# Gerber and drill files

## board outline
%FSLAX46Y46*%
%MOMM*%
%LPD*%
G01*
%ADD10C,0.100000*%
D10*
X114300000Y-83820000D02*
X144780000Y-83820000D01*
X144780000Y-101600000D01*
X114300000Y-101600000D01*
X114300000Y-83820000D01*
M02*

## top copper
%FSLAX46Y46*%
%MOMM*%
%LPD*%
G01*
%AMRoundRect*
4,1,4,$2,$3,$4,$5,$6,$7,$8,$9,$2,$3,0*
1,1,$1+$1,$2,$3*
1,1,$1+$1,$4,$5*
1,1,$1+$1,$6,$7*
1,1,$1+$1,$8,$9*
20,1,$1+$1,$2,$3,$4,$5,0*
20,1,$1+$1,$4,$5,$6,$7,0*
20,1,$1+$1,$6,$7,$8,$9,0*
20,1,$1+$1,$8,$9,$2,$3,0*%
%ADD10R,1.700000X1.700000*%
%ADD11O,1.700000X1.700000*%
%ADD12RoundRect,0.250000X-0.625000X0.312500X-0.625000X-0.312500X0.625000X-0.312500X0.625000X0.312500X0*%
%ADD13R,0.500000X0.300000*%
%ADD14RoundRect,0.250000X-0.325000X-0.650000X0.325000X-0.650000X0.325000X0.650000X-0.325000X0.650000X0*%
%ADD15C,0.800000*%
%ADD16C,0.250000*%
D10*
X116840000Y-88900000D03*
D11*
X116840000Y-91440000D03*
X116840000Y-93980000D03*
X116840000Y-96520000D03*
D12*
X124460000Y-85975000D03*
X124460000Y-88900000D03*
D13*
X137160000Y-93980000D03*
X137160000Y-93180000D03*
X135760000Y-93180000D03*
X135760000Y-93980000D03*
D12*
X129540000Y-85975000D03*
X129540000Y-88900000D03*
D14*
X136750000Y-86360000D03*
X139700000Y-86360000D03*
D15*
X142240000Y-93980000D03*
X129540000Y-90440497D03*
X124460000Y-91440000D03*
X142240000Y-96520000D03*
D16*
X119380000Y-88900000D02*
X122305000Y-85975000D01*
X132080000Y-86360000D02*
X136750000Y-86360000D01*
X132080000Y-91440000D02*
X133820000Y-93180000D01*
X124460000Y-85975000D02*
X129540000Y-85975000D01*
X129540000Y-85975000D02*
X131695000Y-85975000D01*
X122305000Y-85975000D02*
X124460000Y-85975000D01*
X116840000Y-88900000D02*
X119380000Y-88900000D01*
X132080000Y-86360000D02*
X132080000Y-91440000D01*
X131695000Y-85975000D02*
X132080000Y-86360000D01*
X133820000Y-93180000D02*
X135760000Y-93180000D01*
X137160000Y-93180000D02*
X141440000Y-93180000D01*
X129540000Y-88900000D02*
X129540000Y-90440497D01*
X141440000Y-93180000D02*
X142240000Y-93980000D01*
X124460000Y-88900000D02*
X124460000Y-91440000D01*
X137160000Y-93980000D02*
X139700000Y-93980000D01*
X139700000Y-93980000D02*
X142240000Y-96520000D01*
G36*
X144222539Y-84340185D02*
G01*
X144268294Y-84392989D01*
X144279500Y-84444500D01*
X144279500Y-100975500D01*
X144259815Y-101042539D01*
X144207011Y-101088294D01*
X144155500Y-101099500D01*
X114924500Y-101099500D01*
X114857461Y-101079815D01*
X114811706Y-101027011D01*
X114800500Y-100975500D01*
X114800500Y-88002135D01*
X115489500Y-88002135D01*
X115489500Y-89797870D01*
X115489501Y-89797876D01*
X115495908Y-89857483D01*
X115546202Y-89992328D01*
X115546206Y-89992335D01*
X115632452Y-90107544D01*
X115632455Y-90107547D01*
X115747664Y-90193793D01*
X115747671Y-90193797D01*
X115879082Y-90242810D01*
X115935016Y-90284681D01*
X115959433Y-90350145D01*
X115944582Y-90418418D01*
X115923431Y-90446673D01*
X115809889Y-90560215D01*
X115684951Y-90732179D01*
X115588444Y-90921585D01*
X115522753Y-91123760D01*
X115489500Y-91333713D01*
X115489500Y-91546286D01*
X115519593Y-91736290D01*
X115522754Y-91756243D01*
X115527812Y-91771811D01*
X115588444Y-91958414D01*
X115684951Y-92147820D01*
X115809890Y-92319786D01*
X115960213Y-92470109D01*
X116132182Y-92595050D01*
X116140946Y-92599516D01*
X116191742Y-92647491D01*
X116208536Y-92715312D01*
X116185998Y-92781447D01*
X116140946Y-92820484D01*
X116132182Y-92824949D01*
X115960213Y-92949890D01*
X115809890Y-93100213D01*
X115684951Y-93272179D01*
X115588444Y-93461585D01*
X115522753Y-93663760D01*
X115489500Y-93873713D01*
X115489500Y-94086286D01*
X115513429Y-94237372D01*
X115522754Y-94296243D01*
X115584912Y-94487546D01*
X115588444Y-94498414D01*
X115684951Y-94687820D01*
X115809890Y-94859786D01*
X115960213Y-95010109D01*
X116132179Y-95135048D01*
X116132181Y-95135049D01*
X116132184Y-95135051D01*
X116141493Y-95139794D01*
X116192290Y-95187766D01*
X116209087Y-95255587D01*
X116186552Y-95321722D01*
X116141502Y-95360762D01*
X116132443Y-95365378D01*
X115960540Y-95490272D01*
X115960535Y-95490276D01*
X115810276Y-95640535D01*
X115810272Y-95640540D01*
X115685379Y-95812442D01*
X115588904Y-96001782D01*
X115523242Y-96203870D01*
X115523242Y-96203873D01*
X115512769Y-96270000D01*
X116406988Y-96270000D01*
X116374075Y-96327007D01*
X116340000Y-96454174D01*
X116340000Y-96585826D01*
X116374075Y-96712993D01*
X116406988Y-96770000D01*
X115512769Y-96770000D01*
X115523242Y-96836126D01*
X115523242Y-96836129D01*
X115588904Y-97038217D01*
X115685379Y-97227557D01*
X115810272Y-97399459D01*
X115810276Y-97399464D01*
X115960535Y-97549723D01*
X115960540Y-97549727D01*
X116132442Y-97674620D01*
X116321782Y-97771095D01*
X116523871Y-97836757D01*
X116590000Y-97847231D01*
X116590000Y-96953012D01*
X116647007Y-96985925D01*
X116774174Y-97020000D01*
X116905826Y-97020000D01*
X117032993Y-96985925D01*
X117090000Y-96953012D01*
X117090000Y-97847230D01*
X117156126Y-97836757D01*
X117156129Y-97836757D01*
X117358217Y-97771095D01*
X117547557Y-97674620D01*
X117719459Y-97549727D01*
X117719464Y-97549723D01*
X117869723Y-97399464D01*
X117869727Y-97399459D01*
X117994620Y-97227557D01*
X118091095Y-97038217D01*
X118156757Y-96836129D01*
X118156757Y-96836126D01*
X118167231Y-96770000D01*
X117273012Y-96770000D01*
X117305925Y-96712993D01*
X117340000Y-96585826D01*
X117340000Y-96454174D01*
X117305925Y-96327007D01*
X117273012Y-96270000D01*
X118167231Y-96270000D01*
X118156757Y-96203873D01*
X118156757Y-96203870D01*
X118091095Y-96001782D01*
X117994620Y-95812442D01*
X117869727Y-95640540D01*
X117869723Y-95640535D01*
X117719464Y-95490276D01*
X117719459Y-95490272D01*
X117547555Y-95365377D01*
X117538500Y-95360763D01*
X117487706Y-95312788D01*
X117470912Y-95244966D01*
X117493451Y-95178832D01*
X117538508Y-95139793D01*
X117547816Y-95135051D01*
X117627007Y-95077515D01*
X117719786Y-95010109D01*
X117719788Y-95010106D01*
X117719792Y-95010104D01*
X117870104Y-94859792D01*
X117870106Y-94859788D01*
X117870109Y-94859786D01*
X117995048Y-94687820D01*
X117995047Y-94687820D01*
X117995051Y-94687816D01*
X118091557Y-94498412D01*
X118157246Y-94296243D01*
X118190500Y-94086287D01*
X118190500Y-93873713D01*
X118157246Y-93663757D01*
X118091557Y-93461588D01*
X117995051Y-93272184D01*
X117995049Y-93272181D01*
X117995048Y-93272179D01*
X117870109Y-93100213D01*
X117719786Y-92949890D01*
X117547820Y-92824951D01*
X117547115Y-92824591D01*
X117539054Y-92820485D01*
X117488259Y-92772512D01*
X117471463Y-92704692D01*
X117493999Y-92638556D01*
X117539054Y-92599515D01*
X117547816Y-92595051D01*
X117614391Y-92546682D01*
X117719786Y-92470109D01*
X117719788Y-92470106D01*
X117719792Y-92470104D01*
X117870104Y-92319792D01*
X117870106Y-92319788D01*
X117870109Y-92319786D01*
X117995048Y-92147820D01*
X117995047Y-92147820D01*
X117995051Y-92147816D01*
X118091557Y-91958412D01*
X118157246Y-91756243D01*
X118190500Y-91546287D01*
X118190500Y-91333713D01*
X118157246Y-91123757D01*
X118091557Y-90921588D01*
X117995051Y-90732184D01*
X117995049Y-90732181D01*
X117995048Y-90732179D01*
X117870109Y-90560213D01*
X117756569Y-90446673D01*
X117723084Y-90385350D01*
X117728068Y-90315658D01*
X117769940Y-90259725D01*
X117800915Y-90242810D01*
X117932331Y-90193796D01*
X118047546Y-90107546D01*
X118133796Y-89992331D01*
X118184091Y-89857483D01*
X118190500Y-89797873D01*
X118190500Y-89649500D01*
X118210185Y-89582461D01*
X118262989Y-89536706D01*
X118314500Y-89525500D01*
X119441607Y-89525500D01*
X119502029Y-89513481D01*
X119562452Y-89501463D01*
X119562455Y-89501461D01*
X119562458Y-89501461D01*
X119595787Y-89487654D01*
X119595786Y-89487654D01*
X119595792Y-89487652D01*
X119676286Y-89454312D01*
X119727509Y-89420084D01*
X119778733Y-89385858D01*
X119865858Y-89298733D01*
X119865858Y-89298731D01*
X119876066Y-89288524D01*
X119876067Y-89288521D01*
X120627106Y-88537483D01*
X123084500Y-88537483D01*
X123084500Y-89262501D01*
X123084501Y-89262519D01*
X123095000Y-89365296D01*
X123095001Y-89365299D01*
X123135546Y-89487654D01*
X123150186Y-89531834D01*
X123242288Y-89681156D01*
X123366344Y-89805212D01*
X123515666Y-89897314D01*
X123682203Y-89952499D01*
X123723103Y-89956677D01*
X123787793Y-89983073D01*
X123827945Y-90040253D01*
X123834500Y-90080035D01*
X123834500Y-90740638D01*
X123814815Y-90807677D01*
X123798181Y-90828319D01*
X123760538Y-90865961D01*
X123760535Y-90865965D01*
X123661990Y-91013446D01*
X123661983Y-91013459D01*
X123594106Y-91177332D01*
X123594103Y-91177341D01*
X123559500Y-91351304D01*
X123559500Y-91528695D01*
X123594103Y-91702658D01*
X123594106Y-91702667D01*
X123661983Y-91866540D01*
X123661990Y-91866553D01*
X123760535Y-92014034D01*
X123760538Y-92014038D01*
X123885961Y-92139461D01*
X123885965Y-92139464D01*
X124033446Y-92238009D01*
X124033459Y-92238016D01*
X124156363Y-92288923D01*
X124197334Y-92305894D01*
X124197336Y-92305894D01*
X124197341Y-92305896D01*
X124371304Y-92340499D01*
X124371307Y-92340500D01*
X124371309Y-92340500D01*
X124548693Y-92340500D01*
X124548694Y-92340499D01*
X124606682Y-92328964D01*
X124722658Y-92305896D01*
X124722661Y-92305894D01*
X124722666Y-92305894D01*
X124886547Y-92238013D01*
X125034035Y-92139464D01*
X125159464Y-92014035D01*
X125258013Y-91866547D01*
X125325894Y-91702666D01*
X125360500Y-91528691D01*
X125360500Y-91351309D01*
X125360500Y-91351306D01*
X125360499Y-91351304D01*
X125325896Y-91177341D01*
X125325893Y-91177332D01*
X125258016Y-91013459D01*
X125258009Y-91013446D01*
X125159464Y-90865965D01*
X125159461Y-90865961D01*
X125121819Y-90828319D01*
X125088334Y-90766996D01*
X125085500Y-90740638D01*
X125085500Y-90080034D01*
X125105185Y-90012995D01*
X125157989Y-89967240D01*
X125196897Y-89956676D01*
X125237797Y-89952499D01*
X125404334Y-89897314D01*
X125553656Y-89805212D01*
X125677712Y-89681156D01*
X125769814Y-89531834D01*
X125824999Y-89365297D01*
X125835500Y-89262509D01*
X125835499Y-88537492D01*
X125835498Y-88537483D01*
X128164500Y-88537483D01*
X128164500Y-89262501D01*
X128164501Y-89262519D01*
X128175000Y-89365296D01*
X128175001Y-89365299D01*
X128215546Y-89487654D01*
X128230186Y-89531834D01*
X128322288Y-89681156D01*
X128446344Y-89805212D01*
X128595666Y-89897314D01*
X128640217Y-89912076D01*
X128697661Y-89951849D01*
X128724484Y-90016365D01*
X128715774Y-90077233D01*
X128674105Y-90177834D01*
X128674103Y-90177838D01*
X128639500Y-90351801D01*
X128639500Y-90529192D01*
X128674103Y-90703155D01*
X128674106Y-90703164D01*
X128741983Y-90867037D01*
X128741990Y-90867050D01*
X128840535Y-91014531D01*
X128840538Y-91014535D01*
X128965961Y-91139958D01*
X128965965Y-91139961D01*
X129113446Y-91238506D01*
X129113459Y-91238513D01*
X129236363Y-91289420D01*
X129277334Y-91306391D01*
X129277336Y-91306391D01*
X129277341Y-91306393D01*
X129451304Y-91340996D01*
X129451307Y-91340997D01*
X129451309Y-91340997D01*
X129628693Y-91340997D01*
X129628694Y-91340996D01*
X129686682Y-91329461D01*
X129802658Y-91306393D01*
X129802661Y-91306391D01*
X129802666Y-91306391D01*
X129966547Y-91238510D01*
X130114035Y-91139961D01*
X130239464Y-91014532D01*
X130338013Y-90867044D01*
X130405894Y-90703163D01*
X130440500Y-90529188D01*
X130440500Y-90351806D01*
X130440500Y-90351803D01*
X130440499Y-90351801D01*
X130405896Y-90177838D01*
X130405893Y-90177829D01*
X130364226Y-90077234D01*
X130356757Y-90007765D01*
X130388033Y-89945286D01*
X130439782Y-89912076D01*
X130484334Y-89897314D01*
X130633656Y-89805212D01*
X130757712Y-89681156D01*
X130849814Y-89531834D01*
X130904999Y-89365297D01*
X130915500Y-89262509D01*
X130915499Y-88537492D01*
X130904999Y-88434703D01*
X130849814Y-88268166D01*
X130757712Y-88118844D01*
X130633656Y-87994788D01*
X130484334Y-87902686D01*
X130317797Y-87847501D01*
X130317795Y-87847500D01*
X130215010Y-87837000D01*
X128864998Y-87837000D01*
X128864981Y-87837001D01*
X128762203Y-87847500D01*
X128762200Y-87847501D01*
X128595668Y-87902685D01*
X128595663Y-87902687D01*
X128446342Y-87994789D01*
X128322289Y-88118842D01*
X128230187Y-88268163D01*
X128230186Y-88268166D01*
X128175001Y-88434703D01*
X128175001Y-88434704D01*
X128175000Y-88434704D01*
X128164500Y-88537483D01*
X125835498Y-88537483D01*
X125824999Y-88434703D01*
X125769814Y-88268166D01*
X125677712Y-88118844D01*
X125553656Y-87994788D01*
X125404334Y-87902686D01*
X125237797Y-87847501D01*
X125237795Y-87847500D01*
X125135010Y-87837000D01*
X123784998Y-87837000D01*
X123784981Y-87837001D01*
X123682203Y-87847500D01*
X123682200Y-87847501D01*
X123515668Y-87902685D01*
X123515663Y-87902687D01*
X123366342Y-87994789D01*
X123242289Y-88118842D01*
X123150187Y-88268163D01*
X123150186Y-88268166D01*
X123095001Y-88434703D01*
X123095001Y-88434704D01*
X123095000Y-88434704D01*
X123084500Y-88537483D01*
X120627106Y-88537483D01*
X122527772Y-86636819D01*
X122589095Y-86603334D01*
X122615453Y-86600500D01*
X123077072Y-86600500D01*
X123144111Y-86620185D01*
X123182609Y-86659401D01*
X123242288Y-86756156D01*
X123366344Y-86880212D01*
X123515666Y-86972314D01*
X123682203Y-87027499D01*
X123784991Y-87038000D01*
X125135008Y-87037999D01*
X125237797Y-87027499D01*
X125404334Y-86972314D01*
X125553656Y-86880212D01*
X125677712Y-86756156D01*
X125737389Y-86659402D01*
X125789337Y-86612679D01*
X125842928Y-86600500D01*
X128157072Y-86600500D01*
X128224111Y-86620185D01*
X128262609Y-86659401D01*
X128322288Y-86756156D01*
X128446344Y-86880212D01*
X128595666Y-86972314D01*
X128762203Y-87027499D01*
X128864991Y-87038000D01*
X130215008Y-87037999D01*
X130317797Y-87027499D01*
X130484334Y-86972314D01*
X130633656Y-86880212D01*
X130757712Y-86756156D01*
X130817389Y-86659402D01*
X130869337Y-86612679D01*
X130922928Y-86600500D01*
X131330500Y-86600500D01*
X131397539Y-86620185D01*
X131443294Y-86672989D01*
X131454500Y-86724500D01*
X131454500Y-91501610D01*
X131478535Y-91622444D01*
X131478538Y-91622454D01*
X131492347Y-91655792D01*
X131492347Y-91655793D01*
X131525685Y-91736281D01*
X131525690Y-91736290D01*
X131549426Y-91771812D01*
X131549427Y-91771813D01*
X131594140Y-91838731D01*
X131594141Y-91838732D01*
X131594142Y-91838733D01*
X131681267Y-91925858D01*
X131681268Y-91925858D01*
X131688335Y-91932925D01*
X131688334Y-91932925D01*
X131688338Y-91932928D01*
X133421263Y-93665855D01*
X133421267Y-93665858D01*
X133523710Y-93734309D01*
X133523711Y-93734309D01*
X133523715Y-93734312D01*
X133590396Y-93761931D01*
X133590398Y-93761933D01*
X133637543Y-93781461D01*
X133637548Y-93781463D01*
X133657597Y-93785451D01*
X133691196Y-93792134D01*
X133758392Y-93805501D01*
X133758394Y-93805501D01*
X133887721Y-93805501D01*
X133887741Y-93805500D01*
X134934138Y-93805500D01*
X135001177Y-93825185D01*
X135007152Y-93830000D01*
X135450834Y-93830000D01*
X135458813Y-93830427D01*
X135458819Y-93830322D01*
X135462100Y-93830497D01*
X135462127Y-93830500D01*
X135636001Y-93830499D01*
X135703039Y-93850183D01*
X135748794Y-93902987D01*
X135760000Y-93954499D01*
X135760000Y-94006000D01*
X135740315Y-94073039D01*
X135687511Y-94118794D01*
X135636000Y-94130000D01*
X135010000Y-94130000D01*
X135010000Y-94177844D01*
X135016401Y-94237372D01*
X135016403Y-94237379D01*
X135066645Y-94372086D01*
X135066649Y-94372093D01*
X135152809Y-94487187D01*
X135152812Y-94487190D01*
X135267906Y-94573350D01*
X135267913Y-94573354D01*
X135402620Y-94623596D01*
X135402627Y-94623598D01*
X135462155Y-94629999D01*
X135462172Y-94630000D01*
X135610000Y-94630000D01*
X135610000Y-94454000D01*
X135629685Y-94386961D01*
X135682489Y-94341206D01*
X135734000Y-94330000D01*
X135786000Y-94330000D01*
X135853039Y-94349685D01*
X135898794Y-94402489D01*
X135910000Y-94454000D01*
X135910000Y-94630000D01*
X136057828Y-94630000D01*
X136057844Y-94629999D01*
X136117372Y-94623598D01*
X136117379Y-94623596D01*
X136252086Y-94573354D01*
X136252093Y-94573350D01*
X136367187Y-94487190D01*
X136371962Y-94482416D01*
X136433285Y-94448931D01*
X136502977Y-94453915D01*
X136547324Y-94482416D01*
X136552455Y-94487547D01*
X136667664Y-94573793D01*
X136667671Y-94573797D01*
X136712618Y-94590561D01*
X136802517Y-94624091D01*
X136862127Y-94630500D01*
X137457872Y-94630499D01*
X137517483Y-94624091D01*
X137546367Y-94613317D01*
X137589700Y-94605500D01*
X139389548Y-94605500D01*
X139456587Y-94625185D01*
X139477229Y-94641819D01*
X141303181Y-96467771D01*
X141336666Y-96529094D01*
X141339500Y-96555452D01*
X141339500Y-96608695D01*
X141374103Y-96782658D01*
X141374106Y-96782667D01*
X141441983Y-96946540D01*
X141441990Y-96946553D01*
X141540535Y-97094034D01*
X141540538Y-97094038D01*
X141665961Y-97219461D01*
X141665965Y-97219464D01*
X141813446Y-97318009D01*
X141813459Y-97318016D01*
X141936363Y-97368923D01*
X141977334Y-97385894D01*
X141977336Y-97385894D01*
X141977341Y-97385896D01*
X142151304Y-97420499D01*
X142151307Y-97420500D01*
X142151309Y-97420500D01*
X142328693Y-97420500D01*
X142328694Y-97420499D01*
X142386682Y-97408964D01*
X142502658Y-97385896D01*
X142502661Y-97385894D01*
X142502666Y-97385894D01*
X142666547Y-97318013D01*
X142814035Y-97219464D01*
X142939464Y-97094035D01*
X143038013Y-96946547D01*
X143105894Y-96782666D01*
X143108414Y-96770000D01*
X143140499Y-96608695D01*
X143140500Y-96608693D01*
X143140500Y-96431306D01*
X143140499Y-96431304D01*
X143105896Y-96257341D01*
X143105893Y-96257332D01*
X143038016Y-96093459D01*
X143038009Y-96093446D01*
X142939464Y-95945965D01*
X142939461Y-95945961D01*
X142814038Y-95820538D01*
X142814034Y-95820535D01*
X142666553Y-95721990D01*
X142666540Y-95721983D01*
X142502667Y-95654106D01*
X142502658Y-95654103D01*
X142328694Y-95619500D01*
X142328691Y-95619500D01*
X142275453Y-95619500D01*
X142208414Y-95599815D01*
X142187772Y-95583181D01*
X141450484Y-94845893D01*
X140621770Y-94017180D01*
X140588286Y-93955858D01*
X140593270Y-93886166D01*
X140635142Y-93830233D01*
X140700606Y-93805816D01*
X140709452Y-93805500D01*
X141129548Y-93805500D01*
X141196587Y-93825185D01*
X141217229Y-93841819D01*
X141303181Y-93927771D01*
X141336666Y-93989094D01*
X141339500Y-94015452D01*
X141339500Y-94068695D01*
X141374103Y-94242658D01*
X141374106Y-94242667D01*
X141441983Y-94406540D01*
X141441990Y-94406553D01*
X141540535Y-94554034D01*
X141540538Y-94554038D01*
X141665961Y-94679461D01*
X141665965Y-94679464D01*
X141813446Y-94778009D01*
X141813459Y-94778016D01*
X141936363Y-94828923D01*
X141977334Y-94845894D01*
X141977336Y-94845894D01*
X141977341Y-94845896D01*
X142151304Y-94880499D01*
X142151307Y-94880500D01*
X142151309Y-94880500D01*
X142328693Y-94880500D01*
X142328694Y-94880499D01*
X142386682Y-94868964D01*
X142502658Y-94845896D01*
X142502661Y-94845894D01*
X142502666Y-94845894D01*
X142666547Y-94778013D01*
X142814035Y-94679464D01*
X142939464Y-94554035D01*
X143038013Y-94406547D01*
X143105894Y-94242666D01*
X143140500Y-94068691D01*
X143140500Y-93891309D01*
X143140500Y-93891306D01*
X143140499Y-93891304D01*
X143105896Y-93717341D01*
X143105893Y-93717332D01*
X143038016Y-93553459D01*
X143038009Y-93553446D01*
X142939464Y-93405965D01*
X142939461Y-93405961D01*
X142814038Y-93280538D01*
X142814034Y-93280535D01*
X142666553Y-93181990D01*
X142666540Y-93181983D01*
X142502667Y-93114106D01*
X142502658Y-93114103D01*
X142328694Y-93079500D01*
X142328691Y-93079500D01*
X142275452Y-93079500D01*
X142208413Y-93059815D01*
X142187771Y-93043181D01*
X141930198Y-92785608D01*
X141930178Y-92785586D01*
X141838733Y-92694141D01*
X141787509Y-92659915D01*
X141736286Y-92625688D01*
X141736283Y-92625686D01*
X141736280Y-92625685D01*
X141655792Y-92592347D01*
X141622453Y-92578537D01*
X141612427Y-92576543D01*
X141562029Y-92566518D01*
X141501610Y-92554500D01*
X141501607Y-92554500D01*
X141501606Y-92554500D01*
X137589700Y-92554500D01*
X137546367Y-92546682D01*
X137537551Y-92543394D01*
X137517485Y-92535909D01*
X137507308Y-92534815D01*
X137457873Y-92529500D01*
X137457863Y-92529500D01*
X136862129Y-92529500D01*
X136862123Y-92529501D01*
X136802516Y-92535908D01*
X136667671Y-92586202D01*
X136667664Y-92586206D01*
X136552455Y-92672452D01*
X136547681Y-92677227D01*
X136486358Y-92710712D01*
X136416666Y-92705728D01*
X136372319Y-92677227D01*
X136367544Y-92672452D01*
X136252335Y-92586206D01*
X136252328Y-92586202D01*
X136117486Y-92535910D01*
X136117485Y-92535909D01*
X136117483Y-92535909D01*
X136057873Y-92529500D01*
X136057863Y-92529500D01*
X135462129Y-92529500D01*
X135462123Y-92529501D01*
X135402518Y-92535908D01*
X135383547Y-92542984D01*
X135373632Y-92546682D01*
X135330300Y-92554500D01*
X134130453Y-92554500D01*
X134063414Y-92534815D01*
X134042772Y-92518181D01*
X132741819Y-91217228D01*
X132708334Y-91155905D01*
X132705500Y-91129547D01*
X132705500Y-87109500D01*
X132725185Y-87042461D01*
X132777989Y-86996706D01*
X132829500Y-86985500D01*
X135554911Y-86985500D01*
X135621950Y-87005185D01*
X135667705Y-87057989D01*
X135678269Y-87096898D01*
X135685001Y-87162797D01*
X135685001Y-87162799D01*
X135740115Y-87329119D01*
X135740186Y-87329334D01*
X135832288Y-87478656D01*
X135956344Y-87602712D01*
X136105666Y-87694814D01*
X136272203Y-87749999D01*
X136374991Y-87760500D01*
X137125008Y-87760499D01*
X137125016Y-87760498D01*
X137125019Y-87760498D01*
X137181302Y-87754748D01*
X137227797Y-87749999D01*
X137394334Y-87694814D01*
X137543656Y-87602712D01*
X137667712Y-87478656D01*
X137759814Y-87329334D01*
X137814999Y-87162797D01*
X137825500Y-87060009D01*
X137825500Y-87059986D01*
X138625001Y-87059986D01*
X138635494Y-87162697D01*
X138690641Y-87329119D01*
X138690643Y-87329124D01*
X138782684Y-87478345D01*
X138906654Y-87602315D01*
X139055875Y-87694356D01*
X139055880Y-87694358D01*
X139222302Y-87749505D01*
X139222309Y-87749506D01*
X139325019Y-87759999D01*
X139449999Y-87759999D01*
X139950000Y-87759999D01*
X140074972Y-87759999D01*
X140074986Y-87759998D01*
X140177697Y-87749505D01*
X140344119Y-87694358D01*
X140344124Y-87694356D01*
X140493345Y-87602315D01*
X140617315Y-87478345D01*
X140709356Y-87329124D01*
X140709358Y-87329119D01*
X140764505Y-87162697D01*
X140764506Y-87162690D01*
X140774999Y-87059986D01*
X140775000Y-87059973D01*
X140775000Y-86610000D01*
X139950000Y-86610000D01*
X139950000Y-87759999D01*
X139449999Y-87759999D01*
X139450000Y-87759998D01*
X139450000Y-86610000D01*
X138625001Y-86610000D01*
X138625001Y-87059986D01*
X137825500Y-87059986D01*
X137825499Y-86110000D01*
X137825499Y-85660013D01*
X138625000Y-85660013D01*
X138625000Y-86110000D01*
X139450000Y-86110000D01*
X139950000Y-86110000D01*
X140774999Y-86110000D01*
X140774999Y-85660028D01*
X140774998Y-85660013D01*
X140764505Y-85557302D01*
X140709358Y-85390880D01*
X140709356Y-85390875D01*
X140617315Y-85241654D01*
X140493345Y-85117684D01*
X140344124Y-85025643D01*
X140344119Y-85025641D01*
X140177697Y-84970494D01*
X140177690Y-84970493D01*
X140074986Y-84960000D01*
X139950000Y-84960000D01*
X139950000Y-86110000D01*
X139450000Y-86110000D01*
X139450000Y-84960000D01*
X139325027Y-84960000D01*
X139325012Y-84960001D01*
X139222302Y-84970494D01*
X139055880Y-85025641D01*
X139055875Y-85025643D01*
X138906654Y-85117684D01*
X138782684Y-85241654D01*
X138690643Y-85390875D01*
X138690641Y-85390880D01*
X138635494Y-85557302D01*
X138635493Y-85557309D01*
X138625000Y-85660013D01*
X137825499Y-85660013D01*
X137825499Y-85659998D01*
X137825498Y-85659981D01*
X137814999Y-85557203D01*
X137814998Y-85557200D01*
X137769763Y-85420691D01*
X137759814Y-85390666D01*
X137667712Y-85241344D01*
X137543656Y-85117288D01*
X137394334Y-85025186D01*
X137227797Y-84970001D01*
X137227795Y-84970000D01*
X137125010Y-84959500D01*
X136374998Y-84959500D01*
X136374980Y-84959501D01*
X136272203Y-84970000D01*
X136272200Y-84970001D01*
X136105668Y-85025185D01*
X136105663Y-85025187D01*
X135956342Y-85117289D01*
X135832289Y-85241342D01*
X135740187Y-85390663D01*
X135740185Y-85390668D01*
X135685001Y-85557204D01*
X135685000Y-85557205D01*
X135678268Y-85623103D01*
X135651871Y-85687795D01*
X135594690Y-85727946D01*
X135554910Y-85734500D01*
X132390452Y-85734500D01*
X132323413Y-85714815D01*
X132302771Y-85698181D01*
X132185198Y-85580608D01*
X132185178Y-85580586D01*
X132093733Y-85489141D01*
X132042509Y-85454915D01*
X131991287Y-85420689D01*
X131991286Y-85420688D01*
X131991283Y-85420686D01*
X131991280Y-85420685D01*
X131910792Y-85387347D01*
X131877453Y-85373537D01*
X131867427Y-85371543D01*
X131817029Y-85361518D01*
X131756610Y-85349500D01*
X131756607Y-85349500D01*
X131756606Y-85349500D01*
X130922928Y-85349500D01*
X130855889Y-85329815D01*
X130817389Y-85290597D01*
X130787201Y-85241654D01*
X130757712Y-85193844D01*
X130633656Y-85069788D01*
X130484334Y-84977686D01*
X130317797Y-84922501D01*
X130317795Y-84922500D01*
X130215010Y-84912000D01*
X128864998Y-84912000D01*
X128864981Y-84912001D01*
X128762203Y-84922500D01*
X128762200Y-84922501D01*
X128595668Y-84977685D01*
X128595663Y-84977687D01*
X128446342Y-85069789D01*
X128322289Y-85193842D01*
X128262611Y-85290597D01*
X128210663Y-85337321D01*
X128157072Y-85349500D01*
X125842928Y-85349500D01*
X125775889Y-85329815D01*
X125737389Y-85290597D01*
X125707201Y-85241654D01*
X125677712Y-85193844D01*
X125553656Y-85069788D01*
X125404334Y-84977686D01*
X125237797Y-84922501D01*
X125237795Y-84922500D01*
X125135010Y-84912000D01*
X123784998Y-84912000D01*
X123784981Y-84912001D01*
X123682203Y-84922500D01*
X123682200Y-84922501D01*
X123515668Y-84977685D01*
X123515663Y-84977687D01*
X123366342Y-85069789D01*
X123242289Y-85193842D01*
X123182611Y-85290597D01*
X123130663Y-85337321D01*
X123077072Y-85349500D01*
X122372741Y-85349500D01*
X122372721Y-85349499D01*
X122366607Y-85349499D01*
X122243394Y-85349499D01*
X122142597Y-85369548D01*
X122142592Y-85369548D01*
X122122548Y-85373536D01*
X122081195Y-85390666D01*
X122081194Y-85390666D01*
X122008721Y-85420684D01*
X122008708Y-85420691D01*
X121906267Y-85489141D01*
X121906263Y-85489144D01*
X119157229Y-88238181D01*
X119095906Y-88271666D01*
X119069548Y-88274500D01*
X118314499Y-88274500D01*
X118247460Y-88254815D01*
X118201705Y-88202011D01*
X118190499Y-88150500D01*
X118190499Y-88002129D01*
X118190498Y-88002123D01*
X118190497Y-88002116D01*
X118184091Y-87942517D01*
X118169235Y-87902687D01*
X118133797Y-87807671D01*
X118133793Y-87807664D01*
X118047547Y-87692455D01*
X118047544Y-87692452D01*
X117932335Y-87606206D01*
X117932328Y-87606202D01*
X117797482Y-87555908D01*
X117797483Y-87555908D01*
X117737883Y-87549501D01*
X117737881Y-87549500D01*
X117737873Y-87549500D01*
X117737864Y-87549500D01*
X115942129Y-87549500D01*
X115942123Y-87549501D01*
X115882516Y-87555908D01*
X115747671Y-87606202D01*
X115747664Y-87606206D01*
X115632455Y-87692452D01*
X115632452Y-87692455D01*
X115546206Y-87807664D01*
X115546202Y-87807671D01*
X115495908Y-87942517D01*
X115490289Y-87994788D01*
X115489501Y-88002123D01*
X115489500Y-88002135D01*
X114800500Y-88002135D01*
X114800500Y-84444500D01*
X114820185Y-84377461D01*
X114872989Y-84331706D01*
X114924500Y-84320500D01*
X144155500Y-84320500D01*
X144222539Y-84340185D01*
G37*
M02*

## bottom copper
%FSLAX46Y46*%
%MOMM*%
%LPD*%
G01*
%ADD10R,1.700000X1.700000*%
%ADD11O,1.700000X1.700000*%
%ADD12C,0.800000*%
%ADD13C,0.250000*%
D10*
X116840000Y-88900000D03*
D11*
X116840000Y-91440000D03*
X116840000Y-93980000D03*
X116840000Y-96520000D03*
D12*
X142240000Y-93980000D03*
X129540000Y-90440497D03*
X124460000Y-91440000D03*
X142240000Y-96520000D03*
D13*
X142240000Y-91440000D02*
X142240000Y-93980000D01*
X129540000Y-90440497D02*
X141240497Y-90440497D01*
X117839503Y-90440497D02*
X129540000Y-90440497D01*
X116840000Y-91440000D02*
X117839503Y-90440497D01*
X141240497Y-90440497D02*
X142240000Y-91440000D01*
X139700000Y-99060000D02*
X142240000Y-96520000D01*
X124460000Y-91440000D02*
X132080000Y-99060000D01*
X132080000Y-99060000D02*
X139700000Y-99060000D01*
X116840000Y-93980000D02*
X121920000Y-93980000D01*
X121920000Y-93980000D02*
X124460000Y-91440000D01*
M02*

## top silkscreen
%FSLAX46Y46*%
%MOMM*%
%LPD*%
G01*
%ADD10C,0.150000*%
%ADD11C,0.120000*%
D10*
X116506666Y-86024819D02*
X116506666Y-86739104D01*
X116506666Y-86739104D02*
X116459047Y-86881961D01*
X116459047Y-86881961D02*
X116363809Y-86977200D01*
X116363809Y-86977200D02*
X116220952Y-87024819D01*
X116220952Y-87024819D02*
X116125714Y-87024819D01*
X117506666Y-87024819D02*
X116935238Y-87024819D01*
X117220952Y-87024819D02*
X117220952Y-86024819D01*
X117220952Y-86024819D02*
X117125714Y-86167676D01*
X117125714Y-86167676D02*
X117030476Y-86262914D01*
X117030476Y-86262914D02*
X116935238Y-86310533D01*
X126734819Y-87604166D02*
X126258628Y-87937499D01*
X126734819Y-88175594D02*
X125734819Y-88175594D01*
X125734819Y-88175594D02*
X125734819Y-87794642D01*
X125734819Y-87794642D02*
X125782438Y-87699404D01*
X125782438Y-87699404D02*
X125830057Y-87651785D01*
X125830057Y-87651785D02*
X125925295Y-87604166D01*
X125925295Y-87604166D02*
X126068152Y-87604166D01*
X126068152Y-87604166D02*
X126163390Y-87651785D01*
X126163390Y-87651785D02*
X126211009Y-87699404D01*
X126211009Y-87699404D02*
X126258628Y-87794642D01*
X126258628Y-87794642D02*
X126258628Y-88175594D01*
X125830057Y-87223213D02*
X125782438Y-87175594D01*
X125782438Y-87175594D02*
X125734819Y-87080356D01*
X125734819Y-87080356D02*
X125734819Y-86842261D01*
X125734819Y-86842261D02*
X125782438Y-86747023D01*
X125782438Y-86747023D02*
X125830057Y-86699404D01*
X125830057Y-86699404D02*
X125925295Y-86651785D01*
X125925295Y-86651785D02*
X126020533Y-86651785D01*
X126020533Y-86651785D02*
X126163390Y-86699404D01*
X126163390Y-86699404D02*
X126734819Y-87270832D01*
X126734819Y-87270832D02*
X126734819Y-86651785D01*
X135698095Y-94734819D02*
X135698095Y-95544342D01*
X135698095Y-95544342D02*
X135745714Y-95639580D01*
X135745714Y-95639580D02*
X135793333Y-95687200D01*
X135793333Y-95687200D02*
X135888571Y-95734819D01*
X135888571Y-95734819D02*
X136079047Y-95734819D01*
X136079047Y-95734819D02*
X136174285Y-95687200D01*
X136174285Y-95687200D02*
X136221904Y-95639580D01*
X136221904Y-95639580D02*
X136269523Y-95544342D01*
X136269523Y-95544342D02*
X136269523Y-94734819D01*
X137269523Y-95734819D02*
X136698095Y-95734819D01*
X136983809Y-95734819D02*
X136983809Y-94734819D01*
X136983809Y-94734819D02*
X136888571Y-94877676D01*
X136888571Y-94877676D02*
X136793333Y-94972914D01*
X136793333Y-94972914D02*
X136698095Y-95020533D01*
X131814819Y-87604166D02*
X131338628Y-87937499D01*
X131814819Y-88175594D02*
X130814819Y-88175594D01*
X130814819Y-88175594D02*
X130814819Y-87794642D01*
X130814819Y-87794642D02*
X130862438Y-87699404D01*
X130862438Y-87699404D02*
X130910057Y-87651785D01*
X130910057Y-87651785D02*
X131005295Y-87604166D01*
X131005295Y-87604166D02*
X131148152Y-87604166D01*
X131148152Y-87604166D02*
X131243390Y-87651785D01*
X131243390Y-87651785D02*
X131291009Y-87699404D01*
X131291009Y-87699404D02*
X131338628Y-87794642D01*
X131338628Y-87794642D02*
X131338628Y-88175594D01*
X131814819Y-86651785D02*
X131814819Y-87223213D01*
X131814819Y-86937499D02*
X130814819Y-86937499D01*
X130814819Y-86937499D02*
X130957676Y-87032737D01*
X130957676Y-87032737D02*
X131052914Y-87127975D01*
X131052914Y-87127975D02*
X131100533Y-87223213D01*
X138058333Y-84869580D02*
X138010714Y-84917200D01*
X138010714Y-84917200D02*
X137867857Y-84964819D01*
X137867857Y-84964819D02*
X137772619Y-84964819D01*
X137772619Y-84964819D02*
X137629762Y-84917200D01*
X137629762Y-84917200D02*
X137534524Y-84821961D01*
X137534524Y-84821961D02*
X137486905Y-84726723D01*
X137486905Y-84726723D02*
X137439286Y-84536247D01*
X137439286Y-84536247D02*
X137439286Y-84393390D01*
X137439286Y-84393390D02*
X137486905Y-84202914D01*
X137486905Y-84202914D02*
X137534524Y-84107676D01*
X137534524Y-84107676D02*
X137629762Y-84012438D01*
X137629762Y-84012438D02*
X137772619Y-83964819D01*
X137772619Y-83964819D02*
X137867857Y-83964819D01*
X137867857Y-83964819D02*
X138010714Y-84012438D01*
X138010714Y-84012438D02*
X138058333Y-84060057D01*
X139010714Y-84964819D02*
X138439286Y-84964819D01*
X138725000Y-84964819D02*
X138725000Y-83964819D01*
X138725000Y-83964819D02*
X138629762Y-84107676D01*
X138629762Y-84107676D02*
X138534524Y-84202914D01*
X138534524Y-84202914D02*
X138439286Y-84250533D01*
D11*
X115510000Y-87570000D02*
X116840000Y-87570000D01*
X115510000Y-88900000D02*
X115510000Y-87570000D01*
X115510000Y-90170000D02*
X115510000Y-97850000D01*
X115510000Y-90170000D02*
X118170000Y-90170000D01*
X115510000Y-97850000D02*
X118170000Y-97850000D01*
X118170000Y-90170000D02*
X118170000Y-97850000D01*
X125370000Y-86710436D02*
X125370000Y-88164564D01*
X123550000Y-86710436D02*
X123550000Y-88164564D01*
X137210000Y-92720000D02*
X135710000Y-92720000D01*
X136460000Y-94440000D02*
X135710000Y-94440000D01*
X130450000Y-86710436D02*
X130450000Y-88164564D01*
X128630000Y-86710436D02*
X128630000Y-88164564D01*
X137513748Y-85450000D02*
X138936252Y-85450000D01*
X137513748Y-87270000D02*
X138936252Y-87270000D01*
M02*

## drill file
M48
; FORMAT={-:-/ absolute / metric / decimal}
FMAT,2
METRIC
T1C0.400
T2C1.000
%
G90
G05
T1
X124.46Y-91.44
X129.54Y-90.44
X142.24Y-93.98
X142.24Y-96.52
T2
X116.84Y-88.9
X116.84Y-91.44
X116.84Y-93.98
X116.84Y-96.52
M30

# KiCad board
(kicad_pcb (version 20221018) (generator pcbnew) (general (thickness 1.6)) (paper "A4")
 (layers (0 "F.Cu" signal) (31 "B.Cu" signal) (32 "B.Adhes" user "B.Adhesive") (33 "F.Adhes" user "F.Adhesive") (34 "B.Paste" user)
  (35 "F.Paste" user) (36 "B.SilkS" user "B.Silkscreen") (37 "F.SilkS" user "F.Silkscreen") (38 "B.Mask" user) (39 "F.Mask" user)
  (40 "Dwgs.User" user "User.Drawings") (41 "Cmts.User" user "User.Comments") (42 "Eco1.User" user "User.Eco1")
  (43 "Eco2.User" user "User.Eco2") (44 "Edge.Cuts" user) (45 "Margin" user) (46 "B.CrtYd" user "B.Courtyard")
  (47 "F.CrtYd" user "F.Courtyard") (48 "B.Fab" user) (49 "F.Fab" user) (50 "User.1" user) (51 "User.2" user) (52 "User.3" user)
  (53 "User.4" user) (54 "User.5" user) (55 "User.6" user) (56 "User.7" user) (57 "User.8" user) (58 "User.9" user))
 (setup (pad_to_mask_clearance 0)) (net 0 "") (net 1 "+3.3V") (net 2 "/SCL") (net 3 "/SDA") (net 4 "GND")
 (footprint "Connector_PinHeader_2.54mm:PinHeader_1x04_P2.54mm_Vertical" (layer "F.Cu") (at 116.84 88.9)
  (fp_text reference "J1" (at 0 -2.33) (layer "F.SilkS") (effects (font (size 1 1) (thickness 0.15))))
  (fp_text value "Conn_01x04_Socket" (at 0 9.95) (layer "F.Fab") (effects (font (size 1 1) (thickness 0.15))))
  (fp_line (start -1.33 -1.33) (end 0 -1.33) (stroke (width 0.12) (type solid)) (layer "F.SilkS"))
  (fp_line (start -1.33 0) (end -1.33 -1.33) (stroke (width 0.12) (type solid)) (layer "F.SilkS"))
  (fp_line (start -1.33 1.27) (end -1.33 8.95) (stroke (width 0.12) (type solid)) (layer "F.SilkS"))
  (fp_line (start -1.33 1.27) (end 1.33 1.27) (stroke (width 0.12) (type solid)) (layer "F.SilkS"))
  (fp_line (start -1.33 8.95) (end 1.33 8.95) (stroke (width 0.12) (type solid)) (layer "F.SilkS"))
  (fp_line (start 1.33 1.27) (end 1.33 8.95) (stroke (width 0.12) (type solid)) (layer "F.SilkS"))
  (pad "1" thru_hole rect (at 0 0) (size 1.7 1.7) (drill 1) (layers "*.Cu" "*.Mask") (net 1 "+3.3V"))
  (pad "2" thru_hole oval (at 0 2.54) (size 1.7 1.7) (drill 1) (layers "*.Cu" "*.Mask") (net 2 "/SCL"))
  (pad "3" thru_hole oval (at 0 5.08) (size 1.7 1.7) (drill 1) (layers "*.Cu" "*.Mask") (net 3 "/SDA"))
  (pad "4" thru_hole oval (at 0 7.62) (size 1.7 1.7) (drill 1) (layers "*.Cu" "*.Mask") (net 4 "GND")))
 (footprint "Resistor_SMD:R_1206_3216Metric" (layer "F.Cu") (at 124.46 87.4375 -90)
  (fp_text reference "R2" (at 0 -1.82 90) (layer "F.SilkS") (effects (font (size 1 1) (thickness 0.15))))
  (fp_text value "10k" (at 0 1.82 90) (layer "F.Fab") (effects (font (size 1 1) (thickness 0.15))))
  (fp_line (start -0.727064 -0.91) (end 0.727064 -0.91) (stroke (width 0.12) (type solid)) (layer "F.SilkS"))
  (fp_line (start -0.727064 0.91) (end 0.727064 0.91) (stroke (width 0.12) (type solid)) (layer "F.SilkS"))
  (pad "1" smd roundrect (at -1.4625 0 270) (size 1.125 1.75) (layers "F.Cu" "F.Paste" "F.Mask") (roundrect_rratio 0.222222) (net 1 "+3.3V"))
  (pad "2" smd roundrect (at 1.4625 0 270) (size 1.125 1.75) (layers "F.Cu" "F.Paste" "F.Mask") (roundrect_rratio 0.222222) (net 3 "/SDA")))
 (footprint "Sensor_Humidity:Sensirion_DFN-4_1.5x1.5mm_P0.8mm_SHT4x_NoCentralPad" (layer "F.Cu") (at 136.46 93.58 180)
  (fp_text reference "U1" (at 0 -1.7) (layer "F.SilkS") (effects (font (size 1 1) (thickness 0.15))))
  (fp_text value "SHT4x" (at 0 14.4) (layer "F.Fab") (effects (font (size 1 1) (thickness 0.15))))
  (fp_line (start -0.75 0.86) (end 0.75 0.86) (stroke (width 0.12) (type solid)) (layer "F.SilkS"))
  (fp_line (start 0 -0.86) (end 0.75 -0.86) (stroke (width 0.12) (type solid)) (layer "F.SilkS"))
  (pad "1" smd rect (at -0.7 -0.4 180) (size 0.5 0.3) (layers "F.Cu" "F.Paste" "F.Mask") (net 3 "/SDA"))
  (pad "2" smd rect (at -0.7 0.4 180) (size 0.5 0.3) (layers "F.Cu" "F.Paste" "F.Mask") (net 2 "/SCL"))
  (pad "3" smd rect (at 0.7 0.4 180) (size 0.5 0.3) (layers "F.Cu" "F.Paste" "F.Mask") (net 1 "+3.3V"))
  (pad "4" smd rect (at 0.7 -0.4 180) (size 0.5 0.3) (layers "F.Cu" "F.Paste" "F.Mask") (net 4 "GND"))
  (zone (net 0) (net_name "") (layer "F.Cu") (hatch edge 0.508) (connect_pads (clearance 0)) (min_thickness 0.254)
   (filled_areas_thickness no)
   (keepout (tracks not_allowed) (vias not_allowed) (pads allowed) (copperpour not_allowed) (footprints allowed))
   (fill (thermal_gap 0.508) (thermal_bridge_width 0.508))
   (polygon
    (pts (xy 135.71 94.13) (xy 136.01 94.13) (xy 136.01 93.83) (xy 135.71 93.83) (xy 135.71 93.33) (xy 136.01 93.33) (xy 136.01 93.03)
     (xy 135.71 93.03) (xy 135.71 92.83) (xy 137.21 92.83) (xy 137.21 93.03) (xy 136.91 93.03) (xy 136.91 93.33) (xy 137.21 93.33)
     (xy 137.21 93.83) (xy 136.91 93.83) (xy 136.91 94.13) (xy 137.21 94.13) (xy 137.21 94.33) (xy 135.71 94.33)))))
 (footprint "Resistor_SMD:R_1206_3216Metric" (layer "F.Cu") (at 129.54 87.4375 -90)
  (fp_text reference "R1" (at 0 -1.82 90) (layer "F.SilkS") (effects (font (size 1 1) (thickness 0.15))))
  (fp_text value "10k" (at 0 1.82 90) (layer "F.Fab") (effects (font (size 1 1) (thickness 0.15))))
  (fp_line (start -0.727064 -0.91) (end 0.727064 -0.91) (stroke (width 0.12) (type solid)) (layer "F.SilkS"))
  (fp_line (start -0.727064 0.91) (end 0.727064 0.91) (stroke (width 0.12) (type solid)) (layer "F.SilkS"))
  (pad "1" smd roundrect (at -1.4625 0 270) (size 1.125 1.75) (layers "F.Cu" "F.Paste" "F.Mask") (roundrect_rratio 0.222222) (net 1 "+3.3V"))
  (pad "2" smd roundrect (at 1.4625 0 270) (size 1.125 1.75) (layers "F.Cu" "F.Paste" "F.Mask") (roundrect_rratio 0.222222) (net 2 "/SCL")))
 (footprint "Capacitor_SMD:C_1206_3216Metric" (layer "F.Cu") (at 138.225 86.36)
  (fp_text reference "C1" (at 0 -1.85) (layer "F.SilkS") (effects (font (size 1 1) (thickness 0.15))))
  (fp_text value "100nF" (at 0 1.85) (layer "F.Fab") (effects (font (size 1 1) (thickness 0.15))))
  (fp_line (start -0.711252 -0.91) (end 0.711252 -0.91) (stroke (width 0.12) (type solid)) (layer "F.SilkS"))
  (fp_line (start -0.711252 0.91) (end 0.711252 0.91) (stroke (width 0.12) (type solid)) (layer "F.SilkS"))
  (pad "1" smd roundrect (at -1.475 0) (size 1.15 1.8) (layers "F.Cu" "F.Paste" "F.Mask") (roundrect_rratio 0.217391) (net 1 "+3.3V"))
  (pad "2" smd roundrect (at 1.475 0) (size 1.15 1.8) (layers "F.Cu" "F.Paste" "F.Mask") (roundrect_rratio 0.217391) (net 4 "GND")))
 (gr_rect (start 114.3 83.82) (end 144.78 101.6) (stroke (width 0.1) (type default)) (fill none) (layer "Edge.Cuts"))
 (segment (start 119.38 88.9) (end 122.305 85.975) (width 0.25) (layer "F.Cu") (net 1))
 (segment (start 132.08 86.36) (end 136.75 86.36) (width 0.25) (layer "F.Cu") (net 1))
 (segment (start 132.08 91.44) (end 133.82 93.18) (width 0.25) (layer "F.Cu") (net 1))
 (segment (start 124.46 85.975) (end 129.54 85.975) (width 0.25) (layer "F.Cu") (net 1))
 (segment (start 129.54 85.975) (end 131.695 85.975) (width 0.25) (layer "F.Cu") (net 1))
 (segment (start 122.305 85.975) (end 124.46 85.975) (width 0.25) (layer "F.Cu") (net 1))
 (segment (start 116.84 88.9) (end 119.38 88.9) (width 0.25) (layer "F.Cu") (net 1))
 (segment (start 132.08 86.36) (end 132.08 91.44) (width 0.25) (layer "F.Cu") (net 1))
 (segment (start 131.695 85.975) (end 132.08 86.36) (width 0.25) (layer "F.Cu") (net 1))
 (segment (start 133.82 93.18) (end 135.76 93.18) (width 0.25) (layer "F.Cu") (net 1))
 (segment (start 137.16 93.18) (end 141.44 93.18) (width 0.25) (layer "F.Cu") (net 2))
 (segment (start 129.54 88.9) (end 129.54 90.440497) (width 0.25) (layer "F.Cu") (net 2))
 (segment (start 141.44 93.18) (end 142.24 93.98) (width 0.25) (layer "F.Cu") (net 2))
 (via (at 142.24 93.98) (size 0.8) (drill 0.4) (layers "F.Cu" "B.Cu") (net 2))
 (via (at 129.54 90.440497) (size 0.8) (drill 0.4) (layers "F.Cu" "B.Cu") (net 2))
 (segment (start 142.24 91.44) (end 142.24 93.98) (width 0.25) (layer "B.Cu") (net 2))
 (segment (start 129.54 90.440497) (end 141.240497 90.440497) (width 0.25) (layer "B.Cu") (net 2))
 (segment (start 117.839503 90.440497) (end 129.54 90.440497) (width 0.25) (layer "B.Cu") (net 2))
 (segment (start 116.84 91.44) (end 117.839503 90.440497) (width 0.25) (layer "B.Cu") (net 2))
 (segment (start 141.240497 90.440497) (end 142.24 91.44) (width 0.25) (layer "B.Cu") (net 2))
 (segment (start 124.46 88.9) (end 124.46 91.44) (width 0.25) (layer "F.Cu") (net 3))
 (segment (start 137.16 93.98) (end 139.7 93.98) (width 0.25) (layer "F.Cu") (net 3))
 (segment (start 139.7 93.98) (end 142.24 96.52) (width 0.25) (layer "F.Cu") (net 3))
 (via (at 124.46 91.44) (size 0.8) (drill 0.4) (layers "F.Cu" "B.Cu") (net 3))
 (via (at 142.24 96.52) (size 0.8) (drill 0.4) (layers "F.Cu" "B.Cu") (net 3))
 (segment (start 139.7 99.06) (end 142.24 96.52) (width 0.25) (layer "B.Cu") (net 3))
 (segment (start 124.46 91.44) (end 132.08 99.06) (width 0.25) (layer "B.Cu") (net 3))
 (segment (start 132.08 99.06) (end 139.7 99.06) (width 0.25) (layer "B.Cu") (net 3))
 (segment (start 116.84 93.98) (end 121.92 93.98) (width 0.25) (layer "B.Cu") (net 3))
 (segment (start 121.92 93.98) (end 124.46 91.44) (width 0.25) (layer "B.Cu") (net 3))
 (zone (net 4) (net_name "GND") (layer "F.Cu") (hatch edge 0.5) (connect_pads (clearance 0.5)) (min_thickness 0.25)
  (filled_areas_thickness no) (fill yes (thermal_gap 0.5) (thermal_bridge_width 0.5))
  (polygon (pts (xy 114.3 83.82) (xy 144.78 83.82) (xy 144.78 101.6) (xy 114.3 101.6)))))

